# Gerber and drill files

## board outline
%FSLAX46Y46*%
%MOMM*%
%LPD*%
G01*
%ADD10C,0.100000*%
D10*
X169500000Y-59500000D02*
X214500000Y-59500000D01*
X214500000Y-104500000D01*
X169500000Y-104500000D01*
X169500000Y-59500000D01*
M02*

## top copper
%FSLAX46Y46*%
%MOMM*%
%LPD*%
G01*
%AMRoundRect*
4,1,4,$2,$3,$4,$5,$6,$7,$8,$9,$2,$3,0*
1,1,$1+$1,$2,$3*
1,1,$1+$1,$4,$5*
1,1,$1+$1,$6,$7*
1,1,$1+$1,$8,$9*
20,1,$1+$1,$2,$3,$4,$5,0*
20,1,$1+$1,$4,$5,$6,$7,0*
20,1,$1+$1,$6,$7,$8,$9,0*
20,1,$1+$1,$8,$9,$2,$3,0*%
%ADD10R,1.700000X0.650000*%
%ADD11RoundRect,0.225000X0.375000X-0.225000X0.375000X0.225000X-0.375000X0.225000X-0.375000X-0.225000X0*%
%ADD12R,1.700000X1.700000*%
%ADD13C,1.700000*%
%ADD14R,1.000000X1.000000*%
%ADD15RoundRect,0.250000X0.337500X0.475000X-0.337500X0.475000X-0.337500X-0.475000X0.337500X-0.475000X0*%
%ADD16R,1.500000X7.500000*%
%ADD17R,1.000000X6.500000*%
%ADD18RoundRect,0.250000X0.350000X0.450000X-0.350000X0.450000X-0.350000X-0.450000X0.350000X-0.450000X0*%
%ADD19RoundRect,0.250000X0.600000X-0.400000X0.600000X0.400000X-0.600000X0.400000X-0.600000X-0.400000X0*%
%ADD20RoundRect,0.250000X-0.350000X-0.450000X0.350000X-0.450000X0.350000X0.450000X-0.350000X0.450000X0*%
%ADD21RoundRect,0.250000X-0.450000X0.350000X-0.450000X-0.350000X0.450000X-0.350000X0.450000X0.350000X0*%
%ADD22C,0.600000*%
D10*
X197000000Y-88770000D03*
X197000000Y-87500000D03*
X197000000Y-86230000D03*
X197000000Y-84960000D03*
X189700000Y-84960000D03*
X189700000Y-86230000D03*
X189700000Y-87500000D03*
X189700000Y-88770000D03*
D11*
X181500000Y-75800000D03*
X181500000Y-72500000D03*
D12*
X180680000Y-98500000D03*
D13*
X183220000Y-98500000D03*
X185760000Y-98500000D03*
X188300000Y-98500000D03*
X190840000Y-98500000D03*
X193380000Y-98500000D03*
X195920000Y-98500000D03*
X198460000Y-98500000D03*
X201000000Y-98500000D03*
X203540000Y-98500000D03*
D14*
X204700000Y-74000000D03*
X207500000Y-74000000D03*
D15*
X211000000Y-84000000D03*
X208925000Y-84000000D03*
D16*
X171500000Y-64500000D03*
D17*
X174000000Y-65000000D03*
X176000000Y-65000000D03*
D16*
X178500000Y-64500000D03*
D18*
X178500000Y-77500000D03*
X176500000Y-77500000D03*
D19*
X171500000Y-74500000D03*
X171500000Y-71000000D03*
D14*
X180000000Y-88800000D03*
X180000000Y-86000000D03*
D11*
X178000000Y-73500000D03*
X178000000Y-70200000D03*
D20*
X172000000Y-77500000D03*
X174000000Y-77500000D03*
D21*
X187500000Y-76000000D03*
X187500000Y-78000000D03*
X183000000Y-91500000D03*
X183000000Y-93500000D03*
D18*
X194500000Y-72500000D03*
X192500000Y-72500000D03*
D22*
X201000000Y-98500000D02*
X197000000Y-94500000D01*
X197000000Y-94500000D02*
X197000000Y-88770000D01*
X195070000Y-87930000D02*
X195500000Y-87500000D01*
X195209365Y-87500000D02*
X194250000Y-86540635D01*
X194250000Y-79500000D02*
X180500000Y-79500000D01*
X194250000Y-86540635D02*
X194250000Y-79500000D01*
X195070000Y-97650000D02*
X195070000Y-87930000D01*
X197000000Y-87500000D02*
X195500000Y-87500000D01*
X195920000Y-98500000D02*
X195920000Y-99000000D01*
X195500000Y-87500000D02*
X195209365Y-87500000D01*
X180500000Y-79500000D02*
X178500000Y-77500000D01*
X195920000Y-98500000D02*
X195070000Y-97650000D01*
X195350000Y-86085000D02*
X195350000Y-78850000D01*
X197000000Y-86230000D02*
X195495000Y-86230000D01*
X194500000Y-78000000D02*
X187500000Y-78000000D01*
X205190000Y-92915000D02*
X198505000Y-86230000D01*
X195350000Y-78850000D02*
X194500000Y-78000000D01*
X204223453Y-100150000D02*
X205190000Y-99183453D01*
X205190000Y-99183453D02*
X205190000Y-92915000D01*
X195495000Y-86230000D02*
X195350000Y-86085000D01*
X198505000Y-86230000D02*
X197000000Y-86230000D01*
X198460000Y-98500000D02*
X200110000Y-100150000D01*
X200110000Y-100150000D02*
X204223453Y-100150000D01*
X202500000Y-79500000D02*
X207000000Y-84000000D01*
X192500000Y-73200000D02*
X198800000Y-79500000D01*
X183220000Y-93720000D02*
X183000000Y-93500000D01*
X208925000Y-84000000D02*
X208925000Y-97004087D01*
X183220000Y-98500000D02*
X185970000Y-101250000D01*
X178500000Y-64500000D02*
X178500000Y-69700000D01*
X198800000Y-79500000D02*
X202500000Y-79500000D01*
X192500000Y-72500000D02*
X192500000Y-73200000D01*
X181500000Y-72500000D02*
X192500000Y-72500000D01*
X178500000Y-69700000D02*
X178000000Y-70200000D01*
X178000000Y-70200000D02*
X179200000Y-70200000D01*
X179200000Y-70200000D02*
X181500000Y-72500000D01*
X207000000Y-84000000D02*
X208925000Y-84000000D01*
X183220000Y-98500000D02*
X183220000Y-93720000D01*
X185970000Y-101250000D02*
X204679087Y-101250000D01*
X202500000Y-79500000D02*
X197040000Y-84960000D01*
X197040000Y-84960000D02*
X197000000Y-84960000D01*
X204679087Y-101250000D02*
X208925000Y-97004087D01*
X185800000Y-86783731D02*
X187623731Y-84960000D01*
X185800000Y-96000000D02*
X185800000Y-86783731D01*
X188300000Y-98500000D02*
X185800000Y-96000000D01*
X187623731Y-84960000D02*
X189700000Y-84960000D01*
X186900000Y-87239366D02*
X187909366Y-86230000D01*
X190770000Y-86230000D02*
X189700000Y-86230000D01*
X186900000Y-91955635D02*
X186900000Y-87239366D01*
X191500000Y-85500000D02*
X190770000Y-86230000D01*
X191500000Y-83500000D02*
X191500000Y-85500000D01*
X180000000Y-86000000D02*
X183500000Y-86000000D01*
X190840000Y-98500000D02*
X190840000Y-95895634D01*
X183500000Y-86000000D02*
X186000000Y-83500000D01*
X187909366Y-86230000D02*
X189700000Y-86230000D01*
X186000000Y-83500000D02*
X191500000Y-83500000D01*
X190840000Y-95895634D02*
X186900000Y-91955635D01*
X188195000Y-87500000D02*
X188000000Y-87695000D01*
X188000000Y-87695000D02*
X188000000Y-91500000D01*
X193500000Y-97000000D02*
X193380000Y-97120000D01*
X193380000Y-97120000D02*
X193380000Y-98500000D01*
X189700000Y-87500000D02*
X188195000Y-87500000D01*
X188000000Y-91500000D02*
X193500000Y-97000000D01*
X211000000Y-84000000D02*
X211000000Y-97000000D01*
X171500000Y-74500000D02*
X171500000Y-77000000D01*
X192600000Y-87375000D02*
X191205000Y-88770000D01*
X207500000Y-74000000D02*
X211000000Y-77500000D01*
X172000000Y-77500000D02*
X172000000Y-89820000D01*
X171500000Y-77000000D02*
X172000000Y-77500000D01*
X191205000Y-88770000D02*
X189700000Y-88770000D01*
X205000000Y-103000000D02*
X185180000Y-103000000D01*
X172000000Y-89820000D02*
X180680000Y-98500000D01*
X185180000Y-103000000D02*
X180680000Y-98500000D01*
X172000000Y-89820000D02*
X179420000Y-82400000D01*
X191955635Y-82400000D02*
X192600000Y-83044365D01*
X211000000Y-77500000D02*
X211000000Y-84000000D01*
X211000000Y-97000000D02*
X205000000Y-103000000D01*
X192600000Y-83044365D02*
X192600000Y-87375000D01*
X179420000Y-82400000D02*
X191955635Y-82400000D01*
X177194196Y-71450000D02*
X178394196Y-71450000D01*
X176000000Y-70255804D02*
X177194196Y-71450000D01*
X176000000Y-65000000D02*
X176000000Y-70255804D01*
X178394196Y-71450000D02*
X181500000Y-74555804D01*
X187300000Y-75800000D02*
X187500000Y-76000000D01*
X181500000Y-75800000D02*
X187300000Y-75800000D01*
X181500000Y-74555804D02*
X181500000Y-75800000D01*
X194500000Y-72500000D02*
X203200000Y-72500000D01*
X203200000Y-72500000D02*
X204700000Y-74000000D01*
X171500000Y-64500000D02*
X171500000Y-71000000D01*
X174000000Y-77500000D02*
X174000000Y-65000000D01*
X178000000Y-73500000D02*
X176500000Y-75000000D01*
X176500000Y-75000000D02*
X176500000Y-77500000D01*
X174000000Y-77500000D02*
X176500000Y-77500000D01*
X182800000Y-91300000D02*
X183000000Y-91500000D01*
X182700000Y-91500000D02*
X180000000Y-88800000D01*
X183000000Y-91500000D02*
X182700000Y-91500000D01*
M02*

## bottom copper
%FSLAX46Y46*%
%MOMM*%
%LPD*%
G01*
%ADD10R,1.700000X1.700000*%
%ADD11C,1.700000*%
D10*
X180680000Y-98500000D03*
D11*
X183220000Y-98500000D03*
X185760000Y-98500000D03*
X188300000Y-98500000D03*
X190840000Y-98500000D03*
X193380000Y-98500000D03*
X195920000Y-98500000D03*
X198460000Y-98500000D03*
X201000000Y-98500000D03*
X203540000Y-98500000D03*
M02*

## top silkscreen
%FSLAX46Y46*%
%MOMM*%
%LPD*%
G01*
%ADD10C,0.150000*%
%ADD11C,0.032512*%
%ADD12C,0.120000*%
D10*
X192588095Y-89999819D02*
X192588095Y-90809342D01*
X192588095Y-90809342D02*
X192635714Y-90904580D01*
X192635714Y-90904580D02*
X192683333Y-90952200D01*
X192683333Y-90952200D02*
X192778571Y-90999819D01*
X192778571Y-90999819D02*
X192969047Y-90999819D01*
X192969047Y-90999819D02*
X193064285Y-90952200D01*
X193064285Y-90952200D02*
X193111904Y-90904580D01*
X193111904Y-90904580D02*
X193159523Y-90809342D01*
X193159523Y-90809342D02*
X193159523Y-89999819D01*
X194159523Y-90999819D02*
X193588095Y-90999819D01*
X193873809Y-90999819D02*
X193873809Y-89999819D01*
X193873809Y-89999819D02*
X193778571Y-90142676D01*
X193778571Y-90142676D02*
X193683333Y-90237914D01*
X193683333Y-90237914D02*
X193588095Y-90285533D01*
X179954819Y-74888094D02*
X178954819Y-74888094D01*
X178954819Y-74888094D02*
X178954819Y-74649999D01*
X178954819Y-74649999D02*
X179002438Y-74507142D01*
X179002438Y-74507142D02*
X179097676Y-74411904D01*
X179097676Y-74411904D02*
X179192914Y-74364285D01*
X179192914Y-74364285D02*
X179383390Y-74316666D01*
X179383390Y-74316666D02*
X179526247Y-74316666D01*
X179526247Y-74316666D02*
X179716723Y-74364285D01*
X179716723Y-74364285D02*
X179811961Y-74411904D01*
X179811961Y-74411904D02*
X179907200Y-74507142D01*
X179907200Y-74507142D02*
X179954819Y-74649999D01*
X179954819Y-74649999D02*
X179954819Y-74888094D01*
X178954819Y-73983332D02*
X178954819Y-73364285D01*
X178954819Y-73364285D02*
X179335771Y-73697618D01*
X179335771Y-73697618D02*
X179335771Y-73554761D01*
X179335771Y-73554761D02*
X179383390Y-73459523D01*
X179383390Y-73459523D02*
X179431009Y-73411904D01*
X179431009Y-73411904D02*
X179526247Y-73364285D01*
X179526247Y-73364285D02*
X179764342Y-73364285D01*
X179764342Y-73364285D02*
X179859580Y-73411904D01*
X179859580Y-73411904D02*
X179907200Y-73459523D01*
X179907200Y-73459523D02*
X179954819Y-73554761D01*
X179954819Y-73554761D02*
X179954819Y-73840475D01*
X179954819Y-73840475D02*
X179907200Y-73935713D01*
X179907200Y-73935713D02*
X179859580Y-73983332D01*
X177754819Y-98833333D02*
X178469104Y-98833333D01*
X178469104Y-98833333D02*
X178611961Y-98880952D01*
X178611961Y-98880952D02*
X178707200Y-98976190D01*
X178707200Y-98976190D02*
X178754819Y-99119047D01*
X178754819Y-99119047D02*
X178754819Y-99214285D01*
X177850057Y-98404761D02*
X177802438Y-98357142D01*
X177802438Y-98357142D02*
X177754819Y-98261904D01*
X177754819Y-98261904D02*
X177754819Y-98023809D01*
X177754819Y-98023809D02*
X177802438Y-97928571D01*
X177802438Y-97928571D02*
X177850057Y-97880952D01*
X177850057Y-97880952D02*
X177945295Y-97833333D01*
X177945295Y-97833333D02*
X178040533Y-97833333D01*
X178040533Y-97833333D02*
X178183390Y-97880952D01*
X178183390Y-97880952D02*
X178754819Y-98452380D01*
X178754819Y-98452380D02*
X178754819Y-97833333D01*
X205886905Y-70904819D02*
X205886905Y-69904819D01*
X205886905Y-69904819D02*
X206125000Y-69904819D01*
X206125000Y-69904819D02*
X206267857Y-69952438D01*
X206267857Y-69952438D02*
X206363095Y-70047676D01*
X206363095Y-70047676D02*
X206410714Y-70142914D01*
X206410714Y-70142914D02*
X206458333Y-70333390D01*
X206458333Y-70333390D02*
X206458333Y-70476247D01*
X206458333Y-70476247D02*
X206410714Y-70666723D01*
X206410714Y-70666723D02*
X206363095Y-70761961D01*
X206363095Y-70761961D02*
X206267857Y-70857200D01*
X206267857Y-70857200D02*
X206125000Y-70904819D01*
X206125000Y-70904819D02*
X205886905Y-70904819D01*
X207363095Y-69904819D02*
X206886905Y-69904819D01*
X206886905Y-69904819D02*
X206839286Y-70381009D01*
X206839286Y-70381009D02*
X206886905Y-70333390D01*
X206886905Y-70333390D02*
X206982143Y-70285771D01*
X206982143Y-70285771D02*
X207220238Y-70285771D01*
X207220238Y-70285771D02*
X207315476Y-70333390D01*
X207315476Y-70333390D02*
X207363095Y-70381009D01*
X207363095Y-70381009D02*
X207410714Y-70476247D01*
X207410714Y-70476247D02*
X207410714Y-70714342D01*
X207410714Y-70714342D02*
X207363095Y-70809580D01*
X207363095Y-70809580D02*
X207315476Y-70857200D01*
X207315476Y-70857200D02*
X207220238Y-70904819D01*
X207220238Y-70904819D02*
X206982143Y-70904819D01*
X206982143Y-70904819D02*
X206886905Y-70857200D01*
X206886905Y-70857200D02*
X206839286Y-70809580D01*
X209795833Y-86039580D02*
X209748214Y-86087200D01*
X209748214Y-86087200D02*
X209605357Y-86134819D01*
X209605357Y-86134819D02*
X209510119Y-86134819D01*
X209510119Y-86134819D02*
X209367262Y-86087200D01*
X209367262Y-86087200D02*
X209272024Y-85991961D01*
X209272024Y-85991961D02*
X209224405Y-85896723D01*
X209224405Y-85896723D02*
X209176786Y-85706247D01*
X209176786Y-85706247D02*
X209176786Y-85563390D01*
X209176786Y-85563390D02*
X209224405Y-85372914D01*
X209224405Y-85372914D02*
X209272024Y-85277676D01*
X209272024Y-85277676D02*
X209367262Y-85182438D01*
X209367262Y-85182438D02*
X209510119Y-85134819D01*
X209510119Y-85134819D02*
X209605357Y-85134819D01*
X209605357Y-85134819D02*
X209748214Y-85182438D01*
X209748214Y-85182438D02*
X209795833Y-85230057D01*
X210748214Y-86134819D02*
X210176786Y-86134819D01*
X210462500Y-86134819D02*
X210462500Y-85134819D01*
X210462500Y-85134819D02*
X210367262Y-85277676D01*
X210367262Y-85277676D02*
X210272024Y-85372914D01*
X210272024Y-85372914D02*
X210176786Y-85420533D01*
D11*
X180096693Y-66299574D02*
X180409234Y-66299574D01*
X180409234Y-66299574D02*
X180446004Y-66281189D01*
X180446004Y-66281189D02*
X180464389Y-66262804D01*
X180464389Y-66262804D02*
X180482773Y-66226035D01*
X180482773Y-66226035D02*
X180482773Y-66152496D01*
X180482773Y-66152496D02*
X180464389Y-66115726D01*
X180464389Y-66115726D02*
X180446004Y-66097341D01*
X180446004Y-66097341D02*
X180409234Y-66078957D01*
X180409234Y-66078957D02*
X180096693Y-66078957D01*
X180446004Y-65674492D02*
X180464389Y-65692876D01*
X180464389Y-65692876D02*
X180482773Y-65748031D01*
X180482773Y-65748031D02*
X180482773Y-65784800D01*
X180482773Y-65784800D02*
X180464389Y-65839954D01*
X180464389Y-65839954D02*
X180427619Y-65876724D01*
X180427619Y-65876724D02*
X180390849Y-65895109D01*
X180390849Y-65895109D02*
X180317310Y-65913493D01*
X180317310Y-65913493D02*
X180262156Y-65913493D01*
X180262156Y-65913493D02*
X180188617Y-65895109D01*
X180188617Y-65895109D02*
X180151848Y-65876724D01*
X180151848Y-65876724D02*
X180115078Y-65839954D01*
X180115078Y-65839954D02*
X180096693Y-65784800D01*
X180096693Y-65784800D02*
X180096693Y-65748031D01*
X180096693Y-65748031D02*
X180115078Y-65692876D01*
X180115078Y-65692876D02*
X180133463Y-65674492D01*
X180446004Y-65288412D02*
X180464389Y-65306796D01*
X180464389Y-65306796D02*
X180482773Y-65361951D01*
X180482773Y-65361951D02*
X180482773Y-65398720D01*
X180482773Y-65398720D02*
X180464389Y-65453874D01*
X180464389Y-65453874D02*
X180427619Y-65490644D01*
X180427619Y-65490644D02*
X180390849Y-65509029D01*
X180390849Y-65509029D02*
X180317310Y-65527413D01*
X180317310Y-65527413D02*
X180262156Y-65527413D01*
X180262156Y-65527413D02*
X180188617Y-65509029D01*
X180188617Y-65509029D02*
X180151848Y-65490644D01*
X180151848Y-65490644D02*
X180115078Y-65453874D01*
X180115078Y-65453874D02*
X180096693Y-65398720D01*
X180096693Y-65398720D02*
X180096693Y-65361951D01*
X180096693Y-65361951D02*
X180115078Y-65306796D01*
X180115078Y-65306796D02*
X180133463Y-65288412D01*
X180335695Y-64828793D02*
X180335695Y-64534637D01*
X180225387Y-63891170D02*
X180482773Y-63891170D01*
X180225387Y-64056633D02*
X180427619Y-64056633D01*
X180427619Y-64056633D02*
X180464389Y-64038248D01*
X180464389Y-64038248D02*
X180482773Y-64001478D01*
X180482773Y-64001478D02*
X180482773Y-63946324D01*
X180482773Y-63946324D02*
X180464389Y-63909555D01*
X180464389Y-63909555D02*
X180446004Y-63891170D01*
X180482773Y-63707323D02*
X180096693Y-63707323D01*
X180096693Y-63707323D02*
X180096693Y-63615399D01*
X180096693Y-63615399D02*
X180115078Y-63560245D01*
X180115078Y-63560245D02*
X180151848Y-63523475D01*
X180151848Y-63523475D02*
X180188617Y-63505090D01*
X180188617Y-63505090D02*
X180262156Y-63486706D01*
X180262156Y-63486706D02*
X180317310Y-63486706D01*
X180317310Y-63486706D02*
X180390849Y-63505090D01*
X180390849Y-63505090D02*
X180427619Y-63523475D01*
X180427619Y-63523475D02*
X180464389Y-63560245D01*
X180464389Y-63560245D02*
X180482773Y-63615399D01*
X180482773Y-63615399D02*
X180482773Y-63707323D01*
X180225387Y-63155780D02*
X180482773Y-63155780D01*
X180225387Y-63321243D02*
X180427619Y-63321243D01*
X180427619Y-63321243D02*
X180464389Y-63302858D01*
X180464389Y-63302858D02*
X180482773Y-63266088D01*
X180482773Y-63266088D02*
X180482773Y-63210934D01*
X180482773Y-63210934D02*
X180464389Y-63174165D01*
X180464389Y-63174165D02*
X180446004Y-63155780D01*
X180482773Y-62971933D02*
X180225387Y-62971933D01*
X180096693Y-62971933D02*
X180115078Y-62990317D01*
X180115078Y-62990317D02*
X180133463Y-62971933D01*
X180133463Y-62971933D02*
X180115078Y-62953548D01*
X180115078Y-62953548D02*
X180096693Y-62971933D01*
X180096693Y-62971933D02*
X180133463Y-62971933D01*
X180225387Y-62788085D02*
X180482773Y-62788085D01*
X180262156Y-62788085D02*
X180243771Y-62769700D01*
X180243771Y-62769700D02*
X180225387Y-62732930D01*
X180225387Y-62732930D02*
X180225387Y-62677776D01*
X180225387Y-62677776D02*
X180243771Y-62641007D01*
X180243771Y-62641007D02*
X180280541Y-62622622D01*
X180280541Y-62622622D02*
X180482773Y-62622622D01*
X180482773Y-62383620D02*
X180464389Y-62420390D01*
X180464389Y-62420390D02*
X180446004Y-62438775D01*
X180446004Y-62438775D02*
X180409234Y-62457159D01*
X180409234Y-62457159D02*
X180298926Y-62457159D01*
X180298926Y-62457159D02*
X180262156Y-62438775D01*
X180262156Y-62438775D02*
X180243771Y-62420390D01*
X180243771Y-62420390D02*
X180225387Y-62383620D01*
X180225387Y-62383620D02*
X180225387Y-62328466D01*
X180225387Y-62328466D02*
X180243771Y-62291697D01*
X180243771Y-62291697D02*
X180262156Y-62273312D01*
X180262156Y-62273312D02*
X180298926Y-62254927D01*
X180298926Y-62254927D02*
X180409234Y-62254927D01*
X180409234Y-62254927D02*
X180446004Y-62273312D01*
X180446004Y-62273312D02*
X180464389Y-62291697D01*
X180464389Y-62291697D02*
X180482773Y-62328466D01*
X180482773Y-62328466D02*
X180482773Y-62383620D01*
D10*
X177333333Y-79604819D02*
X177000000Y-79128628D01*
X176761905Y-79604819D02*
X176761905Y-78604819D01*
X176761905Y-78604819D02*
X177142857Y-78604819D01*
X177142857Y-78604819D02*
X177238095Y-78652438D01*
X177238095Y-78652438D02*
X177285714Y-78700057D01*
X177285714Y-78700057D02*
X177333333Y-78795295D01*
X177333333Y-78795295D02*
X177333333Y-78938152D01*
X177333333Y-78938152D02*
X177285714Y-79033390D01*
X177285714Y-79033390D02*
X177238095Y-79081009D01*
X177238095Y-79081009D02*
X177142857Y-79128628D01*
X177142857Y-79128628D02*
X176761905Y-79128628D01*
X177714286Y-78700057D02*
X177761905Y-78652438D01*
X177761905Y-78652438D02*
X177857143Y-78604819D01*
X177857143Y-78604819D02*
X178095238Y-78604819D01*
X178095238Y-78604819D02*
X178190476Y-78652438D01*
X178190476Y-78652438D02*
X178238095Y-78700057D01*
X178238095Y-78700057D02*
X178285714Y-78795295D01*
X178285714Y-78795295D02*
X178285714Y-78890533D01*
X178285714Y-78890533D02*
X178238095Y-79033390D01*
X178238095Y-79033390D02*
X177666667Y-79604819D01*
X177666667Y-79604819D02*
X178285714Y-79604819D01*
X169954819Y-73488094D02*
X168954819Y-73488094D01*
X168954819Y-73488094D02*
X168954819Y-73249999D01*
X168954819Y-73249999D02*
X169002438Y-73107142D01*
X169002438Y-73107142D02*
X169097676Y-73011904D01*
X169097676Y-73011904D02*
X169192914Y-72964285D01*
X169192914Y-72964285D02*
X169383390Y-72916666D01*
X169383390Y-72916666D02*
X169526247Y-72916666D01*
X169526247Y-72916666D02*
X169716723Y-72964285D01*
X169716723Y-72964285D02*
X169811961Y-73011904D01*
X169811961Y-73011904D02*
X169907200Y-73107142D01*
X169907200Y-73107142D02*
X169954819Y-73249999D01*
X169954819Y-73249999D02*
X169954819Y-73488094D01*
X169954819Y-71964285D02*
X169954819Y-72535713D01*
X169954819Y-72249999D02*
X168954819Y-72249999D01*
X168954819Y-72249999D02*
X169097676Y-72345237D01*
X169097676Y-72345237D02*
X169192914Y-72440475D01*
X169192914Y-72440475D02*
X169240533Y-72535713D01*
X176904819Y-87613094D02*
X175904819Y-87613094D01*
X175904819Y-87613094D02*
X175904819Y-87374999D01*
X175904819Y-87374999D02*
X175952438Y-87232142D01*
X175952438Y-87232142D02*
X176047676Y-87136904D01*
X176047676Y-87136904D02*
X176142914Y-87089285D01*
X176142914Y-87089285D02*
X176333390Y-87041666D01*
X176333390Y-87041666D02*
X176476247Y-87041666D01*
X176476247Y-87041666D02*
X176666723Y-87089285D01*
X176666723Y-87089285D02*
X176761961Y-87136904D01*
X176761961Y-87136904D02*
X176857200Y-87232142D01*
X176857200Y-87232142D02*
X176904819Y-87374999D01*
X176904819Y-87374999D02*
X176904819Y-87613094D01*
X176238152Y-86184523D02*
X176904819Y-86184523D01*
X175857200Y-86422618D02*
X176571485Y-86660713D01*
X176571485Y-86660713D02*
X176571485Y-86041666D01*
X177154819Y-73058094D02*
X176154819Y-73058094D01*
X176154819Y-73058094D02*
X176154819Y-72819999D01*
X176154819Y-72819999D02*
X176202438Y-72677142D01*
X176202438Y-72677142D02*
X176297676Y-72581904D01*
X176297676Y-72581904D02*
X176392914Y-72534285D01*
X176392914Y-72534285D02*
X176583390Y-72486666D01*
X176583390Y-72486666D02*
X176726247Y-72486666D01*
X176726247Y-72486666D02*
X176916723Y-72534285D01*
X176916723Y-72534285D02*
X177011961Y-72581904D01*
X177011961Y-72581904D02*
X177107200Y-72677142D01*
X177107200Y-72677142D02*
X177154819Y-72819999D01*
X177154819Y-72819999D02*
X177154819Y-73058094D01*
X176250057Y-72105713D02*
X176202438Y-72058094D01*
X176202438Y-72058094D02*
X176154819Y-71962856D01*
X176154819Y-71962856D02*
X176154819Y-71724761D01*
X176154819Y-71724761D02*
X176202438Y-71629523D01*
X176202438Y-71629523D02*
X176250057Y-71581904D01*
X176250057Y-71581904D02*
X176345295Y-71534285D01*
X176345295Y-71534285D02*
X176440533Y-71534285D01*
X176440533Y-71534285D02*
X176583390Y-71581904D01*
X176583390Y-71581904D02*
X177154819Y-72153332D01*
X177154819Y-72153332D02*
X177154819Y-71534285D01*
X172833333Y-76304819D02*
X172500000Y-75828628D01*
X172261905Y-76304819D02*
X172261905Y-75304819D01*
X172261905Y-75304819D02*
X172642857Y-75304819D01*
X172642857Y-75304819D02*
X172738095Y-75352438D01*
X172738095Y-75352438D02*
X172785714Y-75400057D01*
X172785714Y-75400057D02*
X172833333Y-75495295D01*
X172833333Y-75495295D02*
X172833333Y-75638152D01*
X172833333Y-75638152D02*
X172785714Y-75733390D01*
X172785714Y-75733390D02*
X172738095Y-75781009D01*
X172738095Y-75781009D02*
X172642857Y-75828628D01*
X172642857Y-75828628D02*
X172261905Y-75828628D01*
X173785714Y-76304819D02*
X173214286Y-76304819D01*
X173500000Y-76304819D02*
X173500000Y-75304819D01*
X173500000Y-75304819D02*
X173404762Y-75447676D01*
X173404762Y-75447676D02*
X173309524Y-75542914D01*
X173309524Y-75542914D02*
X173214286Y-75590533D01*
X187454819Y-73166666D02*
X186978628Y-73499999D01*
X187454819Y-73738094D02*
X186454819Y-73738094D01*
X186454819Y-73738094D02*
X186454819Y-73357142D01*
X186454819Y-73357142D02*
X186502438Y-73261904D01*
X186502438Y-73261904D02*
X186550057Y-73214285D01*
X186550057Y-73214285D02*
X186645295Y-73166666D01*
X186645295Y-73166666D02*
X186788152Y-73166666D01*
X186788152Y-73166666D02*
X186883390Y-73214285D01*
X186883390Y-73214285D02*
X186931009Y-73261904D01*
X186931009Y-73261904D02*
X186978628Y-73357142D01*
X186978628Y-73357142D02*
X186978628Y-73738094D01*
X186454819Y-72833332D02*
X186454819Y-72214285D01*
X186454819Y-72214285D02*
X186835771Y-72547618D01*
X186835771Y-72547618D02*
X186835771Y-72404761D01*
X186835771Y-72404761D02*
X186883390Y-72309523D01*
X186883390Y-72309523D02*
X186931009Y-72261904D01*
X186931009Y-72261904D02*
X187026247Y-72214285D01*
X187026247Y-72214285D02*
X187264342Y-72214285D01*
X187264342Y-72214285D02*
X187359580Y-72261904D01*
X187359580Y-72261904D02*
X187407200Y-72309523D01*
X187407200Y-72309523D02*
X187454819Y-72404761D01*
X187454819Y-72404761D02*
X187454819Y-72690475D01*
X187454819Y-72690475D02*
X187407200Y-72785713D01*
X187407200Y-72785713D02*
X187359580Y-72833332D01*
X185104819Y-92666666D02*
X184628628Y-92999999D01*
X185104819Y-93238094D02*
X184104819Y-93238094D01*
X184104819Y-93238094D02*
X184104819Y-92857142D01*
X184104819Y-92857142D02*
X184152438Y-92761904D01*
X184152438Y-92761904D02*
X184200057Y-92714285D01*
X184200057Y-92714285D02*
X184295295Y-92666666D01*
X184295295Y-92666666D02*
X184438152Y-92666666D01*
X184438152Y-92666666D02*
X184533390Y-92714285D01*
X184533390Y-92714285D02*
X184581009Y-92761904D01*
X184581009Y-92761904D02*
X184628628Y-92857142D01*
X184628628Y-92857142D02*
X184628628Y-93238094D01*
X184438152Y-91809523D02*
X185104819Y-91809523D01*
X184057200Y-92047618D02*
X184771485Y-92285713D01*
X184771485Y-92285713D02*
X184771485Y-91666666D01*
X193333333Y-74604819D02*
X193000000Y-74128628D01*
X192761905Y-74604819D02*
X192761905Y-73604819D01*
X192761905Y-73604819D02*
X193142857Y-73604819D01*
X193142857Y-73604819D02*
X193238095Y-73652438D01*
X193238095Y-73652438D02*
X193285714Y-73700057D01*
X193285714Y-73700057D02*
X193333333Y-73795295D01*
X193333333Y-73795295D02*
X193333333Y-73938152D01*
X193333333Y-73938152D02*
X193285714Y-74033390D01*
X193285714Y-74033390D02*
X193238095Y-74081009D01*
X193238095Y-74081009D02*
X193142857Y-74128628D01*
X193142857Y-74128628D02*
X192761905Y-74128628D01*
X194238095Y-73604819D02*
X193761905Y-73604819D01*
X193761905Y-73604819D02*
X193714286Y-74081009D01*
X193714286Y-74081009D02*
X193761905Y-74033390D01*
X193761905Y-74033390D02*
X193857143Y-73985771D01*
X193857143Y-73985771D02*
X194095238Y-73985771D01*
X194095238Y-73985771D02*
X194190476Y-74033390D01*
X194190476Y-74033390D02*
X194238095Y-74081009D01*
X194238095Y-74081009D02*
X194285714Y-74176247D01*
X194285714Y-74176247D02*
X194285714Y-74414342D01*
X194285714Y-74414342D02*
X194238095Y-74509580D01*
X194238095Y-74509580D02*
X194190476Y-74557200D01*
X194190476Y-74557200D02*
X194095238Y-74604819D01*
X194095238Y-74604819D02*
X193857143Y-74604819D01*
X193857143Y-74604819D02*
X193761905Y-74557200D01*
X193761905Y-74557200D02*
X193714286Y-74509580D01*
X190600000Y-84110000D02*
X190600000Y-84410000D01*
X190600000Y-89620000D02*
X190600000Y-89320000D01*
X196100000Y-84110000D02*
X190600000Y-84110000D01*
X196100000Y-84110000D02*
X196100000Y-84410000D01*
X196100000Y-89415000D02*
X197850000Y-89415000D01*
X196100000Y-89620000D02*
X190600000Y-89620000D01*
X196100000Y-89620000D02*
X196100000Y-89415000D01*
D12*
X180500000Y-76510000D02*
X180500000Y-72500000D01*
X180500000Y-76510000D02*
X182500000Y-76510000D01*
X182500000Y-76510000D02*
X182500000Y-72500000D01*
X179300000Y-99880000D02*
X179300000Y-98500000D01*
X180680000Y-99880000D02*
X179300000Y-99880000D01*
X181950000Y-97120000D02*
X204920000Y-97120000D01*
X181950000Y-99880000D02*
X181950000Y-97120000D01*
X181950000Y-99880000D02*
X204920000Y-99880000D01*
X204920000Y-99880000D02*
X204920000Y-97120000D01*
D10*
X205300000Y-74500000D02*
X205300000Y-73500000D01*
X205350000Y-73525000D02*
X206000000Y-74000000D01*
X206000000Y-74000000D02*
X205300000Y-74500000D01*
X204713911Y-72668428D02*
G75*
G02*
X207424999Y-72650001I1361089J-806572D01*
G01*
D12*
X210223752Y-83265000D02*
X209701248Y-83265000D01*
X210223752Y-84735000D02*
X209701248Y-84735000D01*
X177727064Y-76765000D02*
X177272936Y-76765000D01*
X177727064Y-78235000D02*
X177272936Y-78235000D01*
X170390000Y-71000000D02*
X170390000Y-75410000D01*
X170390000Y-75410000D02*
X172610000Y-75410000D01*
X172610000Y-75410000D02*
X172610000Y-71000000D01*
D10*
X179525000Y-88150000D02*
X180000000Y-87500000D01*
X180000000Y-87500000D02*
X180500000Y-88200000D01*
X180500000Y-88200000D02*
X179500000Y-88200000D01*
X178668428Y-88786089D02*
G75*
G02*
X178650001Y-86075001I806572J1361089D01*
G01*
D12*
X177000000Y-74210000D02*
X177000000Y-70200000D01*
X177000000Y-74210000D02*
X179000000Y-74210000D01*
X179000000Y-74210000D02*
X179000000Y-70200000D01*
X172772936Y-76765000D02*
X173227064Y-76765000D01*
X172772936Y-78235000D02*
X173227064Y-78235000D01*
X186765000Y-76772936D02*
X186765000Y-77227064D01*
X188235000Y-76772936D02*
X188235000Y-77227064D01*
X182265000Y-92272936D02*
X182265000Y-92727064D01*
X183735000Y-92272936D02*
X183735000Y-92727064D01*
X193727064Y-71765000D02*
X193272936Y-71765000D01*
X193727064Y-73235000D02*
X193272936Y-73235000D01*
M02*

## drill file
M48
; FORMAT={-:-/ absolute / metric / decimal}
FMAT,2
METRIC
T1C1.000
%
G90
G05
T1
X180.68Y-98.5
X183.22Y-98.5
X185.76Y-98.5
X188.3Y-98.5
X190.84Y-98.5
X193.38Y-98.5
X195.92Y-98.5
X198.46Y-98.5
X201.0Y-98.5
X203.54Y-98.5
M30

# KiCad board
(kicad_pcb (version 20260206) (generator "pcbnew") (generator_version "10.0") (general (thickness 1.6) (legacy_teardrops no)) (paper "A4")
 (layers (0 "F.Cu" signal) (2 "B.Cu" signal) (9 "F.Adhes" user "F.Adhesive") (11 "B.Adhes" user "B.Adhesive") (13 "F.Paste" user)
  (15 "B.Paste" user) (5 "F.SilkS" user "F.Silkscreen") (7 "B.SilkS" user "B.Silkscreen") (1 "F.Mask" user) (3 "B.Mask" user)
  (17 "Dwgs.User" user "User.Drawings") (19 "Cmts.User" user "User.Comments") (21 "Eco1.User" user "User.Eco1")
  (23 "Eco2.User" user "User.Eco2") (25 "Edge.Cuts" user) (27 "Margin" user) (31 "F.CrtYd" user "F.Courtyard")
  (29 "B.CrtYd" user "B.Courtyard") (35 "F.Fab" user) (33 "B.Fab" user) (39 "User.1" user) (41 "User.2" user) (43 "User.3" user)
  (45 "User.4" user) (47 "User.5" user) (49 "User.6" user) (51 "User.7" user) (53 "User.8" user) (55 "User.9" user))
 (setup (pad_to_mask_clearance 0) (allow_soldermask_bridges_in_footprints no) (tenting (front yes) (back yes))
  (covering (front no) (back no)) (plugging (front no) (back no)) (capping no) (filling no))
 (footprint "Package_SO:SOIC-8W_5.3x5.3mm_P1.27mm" (layer "F.Cu") (at 193.35 86.865 180)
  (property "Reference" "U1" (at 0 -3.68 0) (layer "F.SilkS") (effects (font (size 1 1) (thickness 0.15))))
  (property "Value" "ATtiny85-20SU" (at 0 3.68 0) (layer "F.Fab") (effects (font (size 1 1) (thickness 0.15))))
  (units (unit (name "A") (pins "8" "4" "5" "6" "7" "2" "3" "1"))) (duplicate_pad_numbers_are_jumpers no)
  (fp_line (start 2.75 2.755) (end 2.75 2.455) (stroke (width 0.15) (type solid)) (layer "F.SilkS"))
  (fp_line (start 2.75 -2.755) (end 2.75 -2.455) (stroke (width 0.15) (type solid)) (layer "F.SilkS"))
  (fp_line (start -2.75 2.755) (end 2.75 2.755) (stroke (width 0.15) (type solid)) (layer "F.SilkS"))
  (fp_line (start -2.75 2.755) (end -2.75 2.455) (stroke (width 0.15) (type solid)) (layer "F.SilkS"))
  (fp_line (start -2.75 -2.55) (end -4.5 -2.55) (stroke (width 0.15) (type solid)) (layer "F.SilkS"))
  (fp_line (start -2.75 -2.755) (end 2.75 -2.755) (stroke (width 0.15) (type solid)) (layer "F.SilkS"))
  (fp_line (start -2.75 -2.755) (end -2.75 -2.55) (stroke (width 0.15) (type solid)) (layer "F.SilkS"))
  (pad "1" smd rect (at -3.65 -1.905 180) (size 1.7 0.65) (layers "F.Cu" "F.Mask" "F.Paste") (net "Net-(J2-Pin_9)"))
  (pad "2" smd rect (at -3.65 -0.635 180) (size 1.7 0.65) (layers "F.Cu" "F.Mask" "F.Paste") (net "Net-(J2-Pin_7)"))
  (pad "3" smd rect (at -3.65 0.635 180) (size 1.7 0.65) (layers "F.Cu" "F.Mask" "F.Paste") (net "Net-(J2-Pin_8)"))
  (pad "4" smd rect (at -3.65 1.905 180) (size 1.7 0.65) (layers "F.Cu" "F.Mask" "F.Paste") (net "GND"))
  (pad "5" smd rect (at 3.65 1.905 180) (size 1.7 0.65) (layers "F.Cu" "F.Mask" "F.Paste") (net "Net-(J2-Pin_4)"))
  (pad "6" smd rect (at 3.65 0.635 180) (size 1.7 0.65) (layers "F.Cu" "F.Mask" "F.Paste") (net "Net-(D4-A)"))
  (pad "7" smd rect (at 3.65 -0.635 180) (size 1.7 0.65) (layers "F.Cu" "F.Mask" "F.Paste") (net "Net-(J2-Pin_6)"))
  (pad "8" smd rect (at 3.65 -1.905 180) (size 1.7 0.65) (layers "F.Cu" "F.Mask" "F.Paste") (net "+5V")))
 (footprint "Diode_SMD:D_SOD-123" (layer "F.Cu") (at 181.5 74.15 90)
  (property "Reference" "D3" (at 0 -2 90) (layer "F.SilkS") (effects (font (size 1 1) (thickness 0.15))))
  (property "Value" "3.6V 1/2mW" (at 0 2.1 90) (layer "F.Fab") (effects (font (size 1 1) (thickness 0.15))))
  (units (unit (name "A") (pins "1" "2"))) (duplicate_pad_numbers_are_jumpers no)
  (fp_line (start -2.36 -1) (end 1.65 -1) (stroke (width 0.12) (type solid)) (layer "F.SilkS"))
  (fp_line (start -2.36 -1) (end -2.36 1) (stroke (width 0.12) (type solid)) (layer "F.SilkS"))
  (fp_line (start -2.36 1) (end 1.65 1) (stroke (width 0.12) (type solid)) (layer "F.SilkS"))
  (pad "1" smd roundrect (at -1.65 0 90) (size 0.9 1.2) (layers "F.Cu" "F.Mask" "F.Paste") (roundrect_rratio 0.25) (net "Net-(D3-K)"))
  (pad "2" smd roundrect (at 1.65 0 90) (size 0.9 1.2) (layers "F.Cu" "F.Mask" "F.Paste") (roundrect_rratio 0.25) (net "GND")))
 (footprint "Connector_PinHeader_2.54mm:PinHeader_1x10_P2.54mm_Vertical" (layer "F.Cu") (at 180.68 98.5 90)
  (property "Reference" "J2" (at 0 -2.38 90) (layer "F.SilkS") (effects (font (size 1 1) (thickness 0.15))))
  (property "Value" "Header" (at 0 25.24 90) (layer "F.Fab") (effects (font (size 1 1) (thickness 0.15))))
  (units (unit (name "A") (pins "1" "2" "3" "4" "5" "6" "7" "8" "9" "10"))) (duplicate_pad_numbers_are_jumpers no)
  (fp_line (start -1.38 -1.38) (end 0 -1.38) (stroke (width 0.12) (type solid)) (layer "F.SilkS"))
  (fp_line (start -1.38 0) (end -1.38 -1.38) (stroke (width 0.12) (type solid)) (layer "F.SilkS"))
  (fp_line (start 1.38 1.27) (end 1.38 24.24) (stroke (width 0.12) (type solid)) (layer "F.SilkS"))
  (fp_line (start -1.38 1.27) (end 1.38 1.27) (stroke (width 0.12) (type solid)) (layer "F.SilkS"))
  (fp_line (start -1.38 1.27) (end -1.38 24.24) (stroke (width 0.12) (type solid)) (layer "F.SilkS"))
  (fp_line (start -1.38 24.24) (end 1.38 24.24) (stroke (width 0.12) (type solid)) (layer "F.SilkS"))
  (pad "1" thru_hole rect (at 0 0 90) (size 1.7 1.7) (drill 1) (layers "*.Cu" "*.Mask") (remove_unused_layers no) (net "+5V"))
  (pad "2" thru_hole circle (at 0 2.54 90) (size 1.7 1.7) (drill 1) (layers "*.Cu" "*.Mask") (remove_unused_layers no) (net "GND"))
  (pad "3" thru_hole circle (at 0 5.08 90) (size 1.7 1.7) (drill 1) (layers "*.Cu" "*.Mask") (remove_unused_layers no)
   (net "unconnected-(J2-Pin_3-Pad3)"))
  (pad "4" thru_hole circle (at 0 7.62 90) (size 1.7 1.7) (drill 1) (layers "*.Cu" "*.Mask") (remove_unused_layers no)
   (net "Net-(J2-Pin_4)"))
  (pad "5" thru_hole circle (at 0 10.16 90) (size 1.7 1.7) (drill 1) (layers "*.Cu" "*.Mask") (remove_unused_layers no) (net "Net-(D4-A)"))
  (pad "6" thru_hole circle (at 0 12.7 90) (size 1.7 1.7) (drill 1) (layers "*.Cu" "*.Mask") (remove_unused_layers no)
   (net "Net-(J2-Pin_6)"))
  (pad "7" thru_hole circle (at 0 15.24 90) (size 1.7 1.7) (drill 1) (layers "*.Cu" "*.Mask") (remove_unused_layers no)
   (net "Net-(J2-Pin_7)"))
  (pad "8" thru_hole circle (at 0 17.78 90) (size 1.7 1.7) (drill 1) (layers "*.Cu" "*.Mask") (remove_unused_layers no)
   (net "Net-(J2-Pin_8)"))
  (pad "9" thru_hole circle (at 0 20.32 90) (size 1.7 1.7) (drill 1) (layers "*.Cu" "*.Mask") (remove_unused_layers no)
   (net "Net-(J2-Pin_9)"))
  (pad "10" thru_hole circle (at 0 22.86 90) (size 1.7 1.7) (drill 1) (layers "*.Cu" "*.Mask") (remove_unused_layers no)
   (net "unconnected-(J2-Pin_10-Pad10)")))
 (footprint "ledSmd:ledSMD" (layer "F.Cu") (at 206.5 74)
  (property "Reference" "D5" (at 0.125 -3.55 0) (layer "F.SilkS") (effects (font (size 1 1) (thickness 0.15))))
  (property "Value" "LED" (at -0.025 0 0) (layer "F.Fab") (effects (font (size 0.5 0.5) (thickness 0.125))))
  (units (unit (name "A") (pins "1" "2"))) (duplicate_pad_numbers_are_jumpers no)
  (fp_line (start -1.2 0.5) (end -1.2 -0.5) (stroke (width 0.15) (type solid)) (layer "F.SilkS"))
  (fp_line (start -1.15 -0.475) (end -0.5 0) (stroke (width 0.15) (type solid)) (layer "F.SilkS"))
  (fp_line (start -0.5 0) (end -1.2 0.5) (stroke (width 0.15) (type solid)) (layer "F.SilkS"))
  (fp_arc (start -1.786089 -1.331572) (mid -0.435753 -2.107089) (end 0.924999 -1.349999) (stroke (width 0.15) (type solid))
   (layer "F.SilkS"))
  (pad "1" smd rect (at -1.8 0) (size 1 1) (layers "F.Cu" "F.Mask" "F.Paste") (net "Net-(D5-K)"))
  (pad "2" smd rect (at 1 0) (size 1 1) (layers "F.Cu" "F.Mask" "F.Paste") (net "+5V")))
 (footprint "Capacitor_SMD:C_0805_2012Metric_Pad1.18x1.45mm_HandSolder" (layer "F.Cu") (at 209.9625 84 180)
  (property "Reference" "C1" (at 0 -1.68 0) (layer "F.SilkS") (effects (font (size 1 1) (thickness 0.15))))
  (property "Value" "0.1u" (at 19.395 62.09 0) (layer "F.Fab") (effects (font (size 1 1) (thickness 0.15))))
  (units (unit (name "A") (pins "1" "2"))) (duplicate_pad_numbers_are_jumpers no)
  (fp_line (start -0.261252 0.735) (end 0.261252 0.735) (stroke (width 0.12) (type solid)) (layer "F.SilkS"))
  (fp_line (start -0.261252 -0.735) (end 0.261252 -0.735) (stroke (width 0.12) (type solid)) (layer "F.SilkS"))
  (pad "1" smd roundrect (at -1.0375 0 180) (size 1.175 1.45) (layers "F.Cu" "F.Mask" "F.Paste") (roundrect_rratio 0.212766) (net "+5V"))
  (pad "2" smd roundrect (at 1.0375 0 180) (size 1.175 1.45) (layers "F.Cu" "F.Mask" "F.Paste") (roundrect_rratio 0.212766) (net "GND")))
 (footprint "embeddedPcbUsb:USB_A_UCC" (layer "F.Cu") (at 175 64.7 -90)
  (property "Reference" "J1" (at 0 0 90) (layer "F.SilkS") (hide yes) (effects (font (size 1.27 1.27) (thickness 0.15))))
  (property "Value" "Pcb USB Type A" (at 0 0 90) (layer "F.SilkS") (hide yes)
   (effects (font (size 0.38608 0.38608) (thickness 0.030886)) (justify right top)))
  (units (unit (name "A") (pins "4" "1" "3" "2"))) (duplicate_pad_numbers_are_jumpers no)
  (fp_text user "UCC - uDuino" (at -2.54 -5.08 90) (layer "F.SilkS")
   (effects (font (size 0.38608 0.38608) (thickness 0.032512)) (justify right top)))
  (pad "1" smd rect (at -0.2 3.5 270) (size 7.5 1.5) (layers "F.Cu" "F.Mask" "F.Paste") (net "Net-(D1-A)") (solder_mask_margin 0.1016))
  (pad "2" smd rect (at 0.3 1 270) (size 6.5 1) (layers "F.Cu" "F.Mask" "F.Paste") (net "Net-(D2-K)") (solder_mask_margin 0.1016))
  (pad "3" smd rect (at 0.3 -1 270) (size 6.5 1) (layers "F.Cu" "F.Mask" "F.Paste") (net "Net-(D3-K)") (solder_mask_margin 0.1016))
  (pad "4" smd rect (at -0.2 -3.5 270) (size 7.5 1.5) (layers "F.Cu" "F.Mask" "F.Paste") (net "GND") (solder_mask_margin 0.1016)))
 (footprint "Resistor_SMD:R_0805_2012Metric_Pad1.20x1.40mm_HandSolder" (layer "F.Cu") (at 177.5 77.5 180)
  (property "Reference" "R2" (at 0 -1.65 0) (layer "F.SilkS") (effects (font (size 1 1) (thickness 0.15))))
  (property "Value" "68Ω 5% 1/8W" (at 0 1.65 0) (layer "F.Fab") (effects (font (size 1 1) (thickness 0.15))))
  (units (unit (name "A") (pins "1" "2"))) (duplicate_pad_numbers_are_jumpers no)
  (fp_line (start -0.227064 0.735) (end 0.227064 0.735) (stroke (width 0.12) (type solid)) (layer "F.SilkS"))
  (fp_line (start -0.227064 -0.735) (end 0.227064 -0.735) (stroke (width 0.12) (type solid)) (layer "F.SilkS"))
  (pad "1" smd roundrect (at -1 0 180) (size 1.2 1.4) (layers "F.Cu" "F.Mask" "F.Paste") (roundrect_rratio 0.208333) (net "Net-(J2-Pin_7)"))
  (pad "2" smd roundrect (at 1 0 180) (size 1.2 1.4) (layers "F.Cu" "F.Mask" "F.Paste") (roundrect_rratio 0.208333) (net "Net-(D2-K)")))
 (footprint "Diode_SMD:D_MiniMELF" (layer "F.Cu") (at 171.5 72.75 90)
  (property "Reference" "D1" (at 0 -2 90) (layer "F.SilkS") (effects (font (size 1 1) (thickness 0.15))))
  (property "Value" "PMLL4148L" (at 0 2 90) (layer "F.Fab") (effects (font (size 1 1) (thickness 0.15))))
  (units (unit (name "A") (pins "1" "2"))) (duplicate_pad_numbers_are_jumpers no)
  (fp_line (start 1.75 -1.11) (end -2.66 -1.11) (stroke (width 0.12) (type solid)) (layer "F.SilkS"))
  (fp_line (start -2.66 -1.11) (end -2.66 1.11) (stroke (width 0.12) (type solid)) (layer "F.SilkS"))
  (fp_line (start -2.66 1.11) (end 1.75 1.11) (stroke (width 0.12) (type solid)) (layer "F.SilkS"))
  (pad "1" smd roundrect (at -1.75 0 90) (size 1.3 1.7) (layers "F.Cu" "F.Mask" "F.Paste") (roundrect_rratio 0.1923076923) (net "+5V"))
  (pad "2" smd roundrect (at 1.75 0 90) (size 1.3 1.7) (layers "F.Cu" "F.Mask" "F.Paste") (roundrect_rratio 0.1923076923) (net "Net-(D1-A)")))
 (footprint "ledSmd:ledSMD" (layer "F.Cu") (at 180 87 90)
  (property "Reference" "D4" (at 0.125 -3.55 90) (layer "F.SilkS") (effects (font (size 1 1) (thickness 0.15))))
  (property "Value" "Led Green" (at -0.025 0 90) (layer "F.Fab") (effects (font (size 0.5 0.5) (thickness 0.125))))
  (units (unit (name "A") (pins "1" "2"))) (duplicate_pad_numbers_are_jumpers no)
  (fp_line (start -1.15 -0.475) (end -0.5 0) (stroke (width 0.15) (type solid)) (layer "F.SilkS"))
  (fp_line (start -0.5 0) (end -1.2 0.5) (stroke (width 0.15) (type solid)) (layer "F.SilkS"))
  (fp_line (start -1.2 0.5) (end -1.2 -0.5) (stroke (width 0.15) (type solid)) (layer "F.SilkS"))
  (fp_arc (start -1.786089 -1.331572) (mid -0.435753 -2.107089) (end 0.924999 -1.349999) (stroke (width 0.15) (type solid))
   (layer "F.SilkS"))
  (pad "1" smd rect (at -1.8 0 90) (size 1 1) (layers "F.Cu" "F.Mask" "F.Paste") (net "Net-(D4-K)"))
  (pad "2" smd rect (at 1 0 90) (size 1 1) (layers "F.Cu" "F.Mask" "F.Paste") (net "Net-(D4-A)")))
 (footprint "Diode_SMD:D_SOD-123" (layer "F.Cu") (at 178 71.85 90)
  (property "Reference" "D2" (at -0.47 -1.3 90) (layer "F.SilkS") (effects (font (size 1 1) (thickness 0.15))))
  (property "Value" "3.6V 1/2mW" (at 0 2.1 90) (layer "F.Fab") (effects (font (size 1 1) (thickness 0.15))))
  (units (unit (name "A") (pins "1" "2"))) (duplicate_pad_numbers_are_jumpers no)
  (fp_line (start -2.36 -1) (end 1.65 -1) (stroke (width 0.12) (type solid)) (layer "F.SilkS"))
  (fp_line (start -2.36 -1) (end -2.36 1) (stroke (width 0.12) (type solid)) (layer "F.SilkS"))
  (fp_line (start -2.36 1) (end 1.65 1) (stroke (width 0.12) (type solid)) (layer "F.SilkS"))
  (pad "1" smd roundrect (at -1.65 0 90) (size 0.9 1.2) (layers "F.Cu" "F.Mask" "F.Paste") (roundrect_rratio 0.25) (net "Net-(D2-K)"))
  (pad "2" smd roundrect (at 1.65 0 90) (size 0.9 1.2) (layers "F.Cu" "F.Mask" "F.Paste") (roundrect_rratio 0.25) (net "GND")))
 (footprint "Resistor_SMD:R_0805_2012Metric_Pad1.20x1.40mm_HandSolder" (layer "F.Cu") (at 173 77.5)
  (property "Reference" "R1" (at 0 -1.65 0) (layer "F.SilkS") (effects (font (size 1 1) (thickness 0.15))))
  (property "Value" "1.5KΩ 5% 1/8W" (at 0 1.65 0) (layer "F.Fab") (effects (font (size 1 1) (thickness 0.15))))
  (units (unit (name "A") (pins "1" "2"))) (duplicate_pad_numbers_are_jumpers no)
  (fp_line (start -0.227064 -0.735) (end 0.227064 -0.735) (stroke (width 0.12) (type solid)) (layer "F.SilkS"))
  (fp_line (start -0.227064 0.735) (end 0.227064 0.735) (stroke (width 0.12) (type solid)) (layer "F.SilkS"))
  (pad "1" smd roundrect (at -1 0) (size 1.2 1.4) (layers "F.Cu" "F.Mask" "F.Paste") (roundrect_rratio 0.208333) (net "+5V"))
  (pad "2" smd roundrect (at 1 0) (size 1.2 1.4) (layers "F.Cu" "F.Mask" "F.Paste") (roundrect_rratio 0.208333) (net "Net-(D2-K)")))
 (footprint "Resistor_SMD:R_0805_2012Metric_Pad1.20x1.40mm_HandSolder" (layer "F.Cu") (at 187.5 77 -90)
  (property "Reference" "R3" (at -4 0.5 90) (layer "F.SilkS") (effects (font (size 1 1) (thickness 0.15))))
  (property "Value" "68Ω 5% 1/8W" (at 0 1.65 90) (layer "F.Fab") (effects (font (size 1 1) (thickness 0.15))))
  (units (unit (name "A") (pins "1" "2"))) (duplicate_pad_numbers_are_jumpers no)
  (fp_line (start -0.227064 0.735) (end 0.227064 0.735) (stroke (width 0.12) (type solid)) (layer "F.SilkS"))
  (fp_line (start -0.227064 -0.735) (end 0.227064 -0.735) (stroke (width 0.12) (type solid)) (layer "F.SilkS"))
  (pad "1" smd roundrect (at -1 0 270) (size 1.2 1.4) (layers "F.Cu" "F.Mask" "F.Paste") (roundrect_rratio 0.208333) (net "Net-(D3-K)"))
  (pad "2" smd roundrect (at 1 0 270) (size 1.2 1.4) (layers "F.Cu" "F.Mask" "F.Paste") (roundrect_rratio 0.208333) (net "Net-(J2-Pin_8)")))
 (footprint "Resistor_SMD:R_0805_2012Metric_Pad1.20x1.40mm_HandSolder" (layer "F.Cu") (at 183 92.5 -90)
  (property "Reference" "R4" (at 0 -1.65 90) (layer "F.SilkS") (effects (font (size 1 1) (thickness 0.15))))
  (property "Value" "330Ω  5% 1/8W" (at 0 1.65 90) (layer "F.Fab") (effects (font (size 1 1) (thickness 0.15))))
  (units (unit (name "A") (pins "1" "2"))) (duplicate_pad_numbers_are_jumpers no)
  (fp_line (start -0.227064 0.735) (end 0.227064 0.735) (stroke (width 0.12) (type solid)) (layer "F.SilkS"))
  (fp_line (start -0.227064 -0.735) (end 0.227064 -0.735) (stroke (width 0.12) (type solid)) (layer "F.SilkS"))
  (pad "1" smd roundrect (at -1 0 270) (size 1.2 1.4) (layers "F.Cu" "F.Mask" "F.Paste") (roundrect_rratio 0.208333) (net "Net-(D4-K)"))
  (pad "2" smd roundrect (at 1 0 270) (size 1.2 1.4) (layers "F.Cu" "F.Mask" "F.Paste") (roundrect_rratio 0.208333) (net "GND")))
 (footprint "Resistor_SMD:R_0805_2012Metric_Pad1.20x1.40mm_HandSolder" (layer "F.Cu") (at 193.5 72.5 180)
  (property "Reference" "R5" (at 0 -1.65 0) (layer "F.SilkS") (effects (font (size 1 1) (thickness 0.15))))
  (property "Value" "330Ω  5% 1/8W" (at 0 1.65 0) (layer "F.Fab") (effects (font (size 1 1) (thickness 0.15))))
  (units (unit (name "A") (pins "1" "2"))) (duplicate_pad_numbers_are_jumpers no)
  (fp_line (start -0.227064 0.735) (end 0.227064 0.735) (stroke (width 0.12) (type solid)) (layer "F.SilkS"))
  (fp_line (start -0.227064 -0.735) (end 0.227064 -0.735) (stroke (width 0.12) (type solid)) (layer "F.SilkS"))
  (pad "1" smd roundrect (at -1 0 180) (size 1.2 1.4) (layers "F.Cu" "F.Mask" "F.Paste") (roundrect_rratio 0.208333) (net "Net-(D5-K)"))
  (pad "2" smd roundrect (at 1 0 180) (size 1.2 1.4) (layers "F.Cu" "F.Mask" "F.Paste") (roundrect_rratio 0.208333) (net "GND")))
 (gr_rect (start 169.5 59.5) (end 214.5 104.5) (stroke (width 0.1) (type default)) (fill no) (layer "Edge.Cuts"))
 (segment (start 201 98.5) (end 197 94.5) (width 0.6) (layer "F.Cu") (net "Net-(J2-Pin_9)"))
 (segment (start 197 94.5) (end 197 88.77) (width 0.6) (layer "F.Cu") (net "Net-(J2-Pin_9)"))
 (segment (start 195.07 87.93) (end 195.5 87.5) (width 0.6) (layer "F.Cu") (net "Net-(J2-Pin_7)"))
 (segment (start 195.209365 87.5) (end 194.25 86.540635) (width 0.6) (layer "F.Cu") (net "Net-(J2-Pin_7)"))
 (segment (start 194.25 79.5) (end 180.5 79.5) (width 0.6) (layer "F.Cu") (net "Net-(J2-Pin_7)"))
 (segment (start 194.25 86.540635) (end 194.25 79.5) (width 0.6) (layer "F.Cu") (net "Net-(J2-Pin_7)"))
 (segment (start 195.07 97.65) (end 195.07 87.93) (width 0.6) (layer "F.Cu") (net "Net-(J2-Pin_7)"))
 (segment (start 197 87.5) (end 195.5 87.5) (width 0.6) (layer "F.Cu") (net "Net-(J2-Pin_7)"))
 (segment (start 195.92 98.5) (end 195.92 99) (width 0.6) (layer "F.Cu") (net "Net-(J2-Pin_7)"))
 (segment (start 195.5 87.5) (end 195.209365 87.5) (width 0.6) (layer "F.Cu") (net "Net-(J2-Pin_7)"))
 (segment (start 180.5 79.5) (end 178.5 77.5) (width 0.6) (layer "F.Cu") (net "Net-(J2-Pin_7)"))
 (segment (start 195.92 98.5) (end 195.07 97.65) (width 0.6) (layer "F.Cu") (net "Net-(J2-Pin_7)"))
 (segment (start 195.35 86.085) (end 195.35 78.85) (width 0.6) (layer "F.Cu") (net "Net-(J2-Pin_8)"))
 (segment (start 197 86.23) (end 195.495 86.23) (width 0.6) (layer "F.Cu") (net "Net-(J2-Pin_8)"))
 (segment (start 194.5 78) (end 187.5 78) (width 0.6) (layer "F.Cu") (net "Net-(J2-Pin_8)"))
 (segment (start 205.19 92.915) (end 198.505 86.23) (width 0.6) (layer "F.Cu") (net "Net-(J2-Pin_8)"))
 (segment (start 195.35 78.85) (end 194.5 78) (width 0.6) (layer "F.Cu") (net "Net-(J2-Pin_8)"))
 (segment (start 204.223453 100.15) (end 205.19 99.183453) (width 0.6) (layer "F.Cu") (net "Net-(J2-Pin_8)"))
 (segment (start 205.19 99.183453) (end 205.19 92.915) (width 0.6) (layer "F.Cu") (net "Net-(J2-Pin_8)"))
 (segment (start 195.495 86.23) (end 195.35 86.085) (width 0.6) (layer "F.Cu") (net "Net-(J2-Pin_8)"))
 (segment (start 198.505 86.23) (end 197 86.23) (width 0.6) (layer "F.Cu") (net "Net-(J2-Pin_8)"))
 (segment (start 198.46 98.5) (end 200.11 100.15) (width 0.6) (layer "F.Cu") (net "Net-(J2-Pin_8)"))
 (segment (start 200.11 100.15) (end 204.223453 100.15) (width 0.6) (layer "F.Cu") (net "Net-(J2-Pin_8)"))
 (segment (start 202.5 79.5) (end 207 84) (width 0.6) (layer "F.Cu") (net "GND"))
 (segment (start 192.5 73.2) (end 198.8 79.5) (width 0.6) (layer "F.Cu") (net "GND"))
 (segment (start 183.22 93.72) (end 183 93.5) (width 0.6) (layer "F.Cu") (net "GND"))
 (segment (start 208.925 84) (end 208.925 97.004087) (width 0.6) (layer "F.Cu") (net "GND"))
 (segment (start 183.22 98.5) (end 185.97 101.25) (width 0.6) (layer "F.Cu") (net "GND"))
 (segment (start 178.5 64.5) (end 178.5 69.7) (width 0.6) (layer "F.Cu") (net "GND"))
 (segment (start 198.8 79.5) (end 202.5 79.5) (width 0.6) (layer "F.Cu") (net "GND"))
 (segment (start 192.5 72.5) (end 192.5 73.2) (width 0.6) (layer "F.Cu") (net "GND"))
 (segment (start 181.5 72.5) (end 192.5 72.5) (width 0.6) (layer "F.Cu") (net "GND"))
 (segment (start 178.5 69.7) (end 178 70.2) (width 0.6) (layer "F.Cu") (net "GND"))
 (segment (start 178 70.2) (end 179.2 70.2) (width 0.6) (layer "F.Cu") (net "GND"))
 (segment (start 179.2 70.2) (end 181.5 72.5) (width 0.6) (layer "F.Cu") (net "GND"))
 (segment (start 207 84) (end 208.925 84) (width 0.6) (layer "F.Cu") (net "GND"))
 (segment (start 183.22 98.5) (end 183.22 93.72) (width 0.6) (layer "F.Cu") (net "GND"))
 (segment (start 185.97 101.25) (end 204.679087 101.25) (width 0.6) (layer "F.Cu") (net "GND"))
 (segment (start 202.5 79.5) (end 197.04 84.96) (width 0.6) (layer "F.Cu") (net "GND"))
 (segment (start 197.04 84.96) (end 197 84.96) (width 0.6) (layer "F.Cu") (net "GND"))
 (segment (start 204.679087 101.25) (end 208.925 97.004087) (width 0.6) (layer "F.Cu") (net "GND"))
 (segment (start 185.8 86.783731) (end 187.623731 84.96) (width 0.6) (layer "F.Cu") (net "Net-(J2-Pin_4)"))
 (segment (start 185.8 96) (end 185.8 86.783731) (width 0.6) (layer "F.Cu") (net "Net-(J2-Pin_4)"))
 (segment (start 188.3 98.5) (end 185.8 96) (width 0.6) (layer "F.Cu") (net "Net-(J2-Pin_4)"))
 (segment (start 187.623731 84.96) (end 189.7 84.96) (width 0.6) (layer "F.Cu") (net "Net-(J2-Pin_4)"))
 (segment (start 186.9 87.239366) (end 187.909366 86.23) (width 0.6) (layer "F.Cu") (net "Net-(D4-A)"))
 (segment (start 190.77 86.23) (end 189.7 86.23) (width 0.6) (layer "F.Cu") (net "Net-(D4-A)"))
 (segment (start 186.9 91.955635) (end 186.9 87.239366) (width 0.6) (layer "F.Cu") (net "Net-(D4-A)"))
 (segment (start 191.5 85.5) (end 190.77 86.23) (width 0.6) (layer "F.Cu") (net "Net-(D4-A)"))
 (segment (start 191.5 83.5) (end 191.5 85.5) (width 0.6) (layer "F.Cu") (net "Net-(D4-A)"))
 (segment (start 180 86) (end 183.5 86) (width 0.6) (layer "F.Cu") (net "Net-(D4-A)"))
 (segment (start 190.84 98.5) (end 190.84 95.895634) (width 0.6) (layer "F.Cu") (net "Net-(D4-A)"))
 (segment (start 183.5 86) (end 186 83.5) (width 0.6) (layer "F.Cu") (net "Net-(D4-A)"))
 (segment (start 187.909366 86.23) (end 189.7 86.23) (width 0.6) (layer "F.Cu") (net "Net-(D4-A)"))
 (segment (start 186 83.5) (end 191.5 83.5) (width 0.6) (layer "F.Cu") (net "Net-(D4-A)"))
 (segment (start 190.84 95.895634) (end 186.9 91.955635) (width 0.6) (layer "F.Cu") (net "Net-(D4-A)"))
 (segment (start 188.195 87.5) (end 188 87.695) (width 0.6) (layer "F.Cu") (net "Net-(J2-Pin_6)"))
 (segment (start 188 87.695) (end 188 91.5) (width 0.6) (layer "F.Cu") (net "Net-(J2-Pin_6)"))
 (segment (start 193.5 97) (end 193.38 97.12) (width 0.6) (layer "F.Cu") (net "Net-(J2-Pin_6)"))
 (segment (start 193.38 97.12) (end 193.38 98.5) (width 0.6) (layer "F.Cu") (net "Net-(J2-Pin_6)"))
 (segment (start 189.7 87.5) (end 188.195 87.5) (width 0.6) (layer "F.Cu") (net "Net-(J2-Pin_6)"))
 (segment (start 188 91.5) (end 193.5 97) (width 0.6) (layer "F.Cu") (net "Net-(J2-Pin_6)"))
 (segment (start 211 84) (end 211 97) (width 0.6) (layer "F.Cu") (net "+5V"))
 (segment (start 171.5 74.5) (end 171.5 77) (width 0.6) (layer "F.Cu") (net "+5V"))
 (segment (start 192.6 87.375) (end 191.205 88.77) (width 0.6) (layer "F.Cu") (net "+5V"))
 (segment (start 207.5 74) (end 211 77.5) (width 0.6) (layer "F.Cu") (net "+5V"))
 (segment (start 172 77.5) (end 172 89.82) (width 0.6) (layer "F.Cu") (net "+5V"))
 (segment (start 171.5 77) (end 172 77.5) (width 0.6) (layer "F.Cu") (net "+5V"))
 (segment (start 191.205 88.77) (end 189.7 88.77) (width 0.6) (layer "F.Cu") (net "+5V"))
 (segment (start 205 103) (end 185.18 103) (width 0.6) (layer "F.Cu") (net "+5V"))
 (segment (start 172 89.82) (end 180.68 98.5) (width 0.6) (layer "F.Cu") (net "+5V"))
 (segment (start 185.18 103) (end 180.68 98.5) (width 0.6) (layer "F.Cu") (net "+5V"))
 (segment (start 172 89.82) (end 179.42 82.4) (width 0.6) (layer "F.Cu") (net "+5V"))
 (segment (start 191.955635 82.4) (end 192.6 83.044365) (width 0.6) (layer "F.Cu") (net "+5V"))
 (segment (start 211 77.5) (end 211 84) (width 0.6) (layer "F.Cu") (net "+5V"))
 (segment (start 211 97) (end 205 103) (width 0.6) (layer "F.Cu") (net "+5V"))
 (segment (start 192.6 83.044365) (end 192.6 87.375) (width 0.6) (layer "F.Cu") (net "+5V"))
 (segment (start 179.42 82.4) (end 191.955635 82.4) (width 0.6) (layer "F.Cu") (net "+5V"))
 (segment (start 177.194196 71.45) (end 178.394196 71.45) (width 0.6) (layer "F.Cu") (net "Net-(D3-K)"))
 (segment (start 176 70.255804) (end 177.194196 71.45) (width 0.6) (layer "F.Cu") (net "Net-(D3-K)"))
 (segment (start 176 65) (end 176 70.255804) (width 0.6) (layer "F.Cu") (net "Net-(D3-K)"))
 (segment (start 178.394196 71.45) (end 181.5 74.555804) (width 0.6) (layer "F.Cu") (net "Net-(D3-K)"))
 (segment (start 187.3 75.8) (end 187.5 76) (width 0.6) (layer "F.Cu") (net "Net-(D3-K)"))
 (segment (start 181.5 75.8) (end 187.3 75.8) (width 0.6) (layer "F.Cu") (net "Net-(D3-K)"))
 (segment (start 181.5 74.555804) (end 181.5 75.8) (width 0.6) (layer "F.Cu") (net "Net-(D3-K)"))
 (segment (start 194.5 72.5) (end 203.2 72.5) (width 0.6) (layer "F.Cu") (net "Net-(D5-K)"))
 (segment (start 203.2 72.5) (end 204.7 74) (width 0.6) (layer "F.Cu") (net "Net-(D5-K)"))
 (segment (start 171.5 64.5) (end 171.5 71) (width 0.6) (layer "F.Cu") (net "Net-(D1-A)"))
 (segment (start 174 77.5) (end 174 65) (width 0.6) (layer "F.Cu") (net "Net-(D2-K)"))
 (segment (start 178 73.5) (end 176.5 75) (width 0.6) (layer "F.Cu") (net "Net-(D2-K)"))
 (segment (start 176.5 75) (end 176.5 77.5) (width 0.6) (layer "F.Cu") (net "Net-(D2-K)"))
 (segment (start 174 77.5) (end 176.5 77.5) (width 0.6) (layer "F.Cu") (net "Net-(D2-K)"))
 (segment (start 182.8 91.3) (end 183 91.5) (width 0.6) (layer "F.Cu") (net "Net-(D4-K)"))
 (segment (start 182.7 91.5) (end 180 88.8) (width 0.6) (layer "F.Cu") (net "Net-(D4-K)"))
 (segment (start 183 91.5) (end 182.7 91.5) (width 0.6) (layer "F.Cu") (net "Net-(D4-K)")))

